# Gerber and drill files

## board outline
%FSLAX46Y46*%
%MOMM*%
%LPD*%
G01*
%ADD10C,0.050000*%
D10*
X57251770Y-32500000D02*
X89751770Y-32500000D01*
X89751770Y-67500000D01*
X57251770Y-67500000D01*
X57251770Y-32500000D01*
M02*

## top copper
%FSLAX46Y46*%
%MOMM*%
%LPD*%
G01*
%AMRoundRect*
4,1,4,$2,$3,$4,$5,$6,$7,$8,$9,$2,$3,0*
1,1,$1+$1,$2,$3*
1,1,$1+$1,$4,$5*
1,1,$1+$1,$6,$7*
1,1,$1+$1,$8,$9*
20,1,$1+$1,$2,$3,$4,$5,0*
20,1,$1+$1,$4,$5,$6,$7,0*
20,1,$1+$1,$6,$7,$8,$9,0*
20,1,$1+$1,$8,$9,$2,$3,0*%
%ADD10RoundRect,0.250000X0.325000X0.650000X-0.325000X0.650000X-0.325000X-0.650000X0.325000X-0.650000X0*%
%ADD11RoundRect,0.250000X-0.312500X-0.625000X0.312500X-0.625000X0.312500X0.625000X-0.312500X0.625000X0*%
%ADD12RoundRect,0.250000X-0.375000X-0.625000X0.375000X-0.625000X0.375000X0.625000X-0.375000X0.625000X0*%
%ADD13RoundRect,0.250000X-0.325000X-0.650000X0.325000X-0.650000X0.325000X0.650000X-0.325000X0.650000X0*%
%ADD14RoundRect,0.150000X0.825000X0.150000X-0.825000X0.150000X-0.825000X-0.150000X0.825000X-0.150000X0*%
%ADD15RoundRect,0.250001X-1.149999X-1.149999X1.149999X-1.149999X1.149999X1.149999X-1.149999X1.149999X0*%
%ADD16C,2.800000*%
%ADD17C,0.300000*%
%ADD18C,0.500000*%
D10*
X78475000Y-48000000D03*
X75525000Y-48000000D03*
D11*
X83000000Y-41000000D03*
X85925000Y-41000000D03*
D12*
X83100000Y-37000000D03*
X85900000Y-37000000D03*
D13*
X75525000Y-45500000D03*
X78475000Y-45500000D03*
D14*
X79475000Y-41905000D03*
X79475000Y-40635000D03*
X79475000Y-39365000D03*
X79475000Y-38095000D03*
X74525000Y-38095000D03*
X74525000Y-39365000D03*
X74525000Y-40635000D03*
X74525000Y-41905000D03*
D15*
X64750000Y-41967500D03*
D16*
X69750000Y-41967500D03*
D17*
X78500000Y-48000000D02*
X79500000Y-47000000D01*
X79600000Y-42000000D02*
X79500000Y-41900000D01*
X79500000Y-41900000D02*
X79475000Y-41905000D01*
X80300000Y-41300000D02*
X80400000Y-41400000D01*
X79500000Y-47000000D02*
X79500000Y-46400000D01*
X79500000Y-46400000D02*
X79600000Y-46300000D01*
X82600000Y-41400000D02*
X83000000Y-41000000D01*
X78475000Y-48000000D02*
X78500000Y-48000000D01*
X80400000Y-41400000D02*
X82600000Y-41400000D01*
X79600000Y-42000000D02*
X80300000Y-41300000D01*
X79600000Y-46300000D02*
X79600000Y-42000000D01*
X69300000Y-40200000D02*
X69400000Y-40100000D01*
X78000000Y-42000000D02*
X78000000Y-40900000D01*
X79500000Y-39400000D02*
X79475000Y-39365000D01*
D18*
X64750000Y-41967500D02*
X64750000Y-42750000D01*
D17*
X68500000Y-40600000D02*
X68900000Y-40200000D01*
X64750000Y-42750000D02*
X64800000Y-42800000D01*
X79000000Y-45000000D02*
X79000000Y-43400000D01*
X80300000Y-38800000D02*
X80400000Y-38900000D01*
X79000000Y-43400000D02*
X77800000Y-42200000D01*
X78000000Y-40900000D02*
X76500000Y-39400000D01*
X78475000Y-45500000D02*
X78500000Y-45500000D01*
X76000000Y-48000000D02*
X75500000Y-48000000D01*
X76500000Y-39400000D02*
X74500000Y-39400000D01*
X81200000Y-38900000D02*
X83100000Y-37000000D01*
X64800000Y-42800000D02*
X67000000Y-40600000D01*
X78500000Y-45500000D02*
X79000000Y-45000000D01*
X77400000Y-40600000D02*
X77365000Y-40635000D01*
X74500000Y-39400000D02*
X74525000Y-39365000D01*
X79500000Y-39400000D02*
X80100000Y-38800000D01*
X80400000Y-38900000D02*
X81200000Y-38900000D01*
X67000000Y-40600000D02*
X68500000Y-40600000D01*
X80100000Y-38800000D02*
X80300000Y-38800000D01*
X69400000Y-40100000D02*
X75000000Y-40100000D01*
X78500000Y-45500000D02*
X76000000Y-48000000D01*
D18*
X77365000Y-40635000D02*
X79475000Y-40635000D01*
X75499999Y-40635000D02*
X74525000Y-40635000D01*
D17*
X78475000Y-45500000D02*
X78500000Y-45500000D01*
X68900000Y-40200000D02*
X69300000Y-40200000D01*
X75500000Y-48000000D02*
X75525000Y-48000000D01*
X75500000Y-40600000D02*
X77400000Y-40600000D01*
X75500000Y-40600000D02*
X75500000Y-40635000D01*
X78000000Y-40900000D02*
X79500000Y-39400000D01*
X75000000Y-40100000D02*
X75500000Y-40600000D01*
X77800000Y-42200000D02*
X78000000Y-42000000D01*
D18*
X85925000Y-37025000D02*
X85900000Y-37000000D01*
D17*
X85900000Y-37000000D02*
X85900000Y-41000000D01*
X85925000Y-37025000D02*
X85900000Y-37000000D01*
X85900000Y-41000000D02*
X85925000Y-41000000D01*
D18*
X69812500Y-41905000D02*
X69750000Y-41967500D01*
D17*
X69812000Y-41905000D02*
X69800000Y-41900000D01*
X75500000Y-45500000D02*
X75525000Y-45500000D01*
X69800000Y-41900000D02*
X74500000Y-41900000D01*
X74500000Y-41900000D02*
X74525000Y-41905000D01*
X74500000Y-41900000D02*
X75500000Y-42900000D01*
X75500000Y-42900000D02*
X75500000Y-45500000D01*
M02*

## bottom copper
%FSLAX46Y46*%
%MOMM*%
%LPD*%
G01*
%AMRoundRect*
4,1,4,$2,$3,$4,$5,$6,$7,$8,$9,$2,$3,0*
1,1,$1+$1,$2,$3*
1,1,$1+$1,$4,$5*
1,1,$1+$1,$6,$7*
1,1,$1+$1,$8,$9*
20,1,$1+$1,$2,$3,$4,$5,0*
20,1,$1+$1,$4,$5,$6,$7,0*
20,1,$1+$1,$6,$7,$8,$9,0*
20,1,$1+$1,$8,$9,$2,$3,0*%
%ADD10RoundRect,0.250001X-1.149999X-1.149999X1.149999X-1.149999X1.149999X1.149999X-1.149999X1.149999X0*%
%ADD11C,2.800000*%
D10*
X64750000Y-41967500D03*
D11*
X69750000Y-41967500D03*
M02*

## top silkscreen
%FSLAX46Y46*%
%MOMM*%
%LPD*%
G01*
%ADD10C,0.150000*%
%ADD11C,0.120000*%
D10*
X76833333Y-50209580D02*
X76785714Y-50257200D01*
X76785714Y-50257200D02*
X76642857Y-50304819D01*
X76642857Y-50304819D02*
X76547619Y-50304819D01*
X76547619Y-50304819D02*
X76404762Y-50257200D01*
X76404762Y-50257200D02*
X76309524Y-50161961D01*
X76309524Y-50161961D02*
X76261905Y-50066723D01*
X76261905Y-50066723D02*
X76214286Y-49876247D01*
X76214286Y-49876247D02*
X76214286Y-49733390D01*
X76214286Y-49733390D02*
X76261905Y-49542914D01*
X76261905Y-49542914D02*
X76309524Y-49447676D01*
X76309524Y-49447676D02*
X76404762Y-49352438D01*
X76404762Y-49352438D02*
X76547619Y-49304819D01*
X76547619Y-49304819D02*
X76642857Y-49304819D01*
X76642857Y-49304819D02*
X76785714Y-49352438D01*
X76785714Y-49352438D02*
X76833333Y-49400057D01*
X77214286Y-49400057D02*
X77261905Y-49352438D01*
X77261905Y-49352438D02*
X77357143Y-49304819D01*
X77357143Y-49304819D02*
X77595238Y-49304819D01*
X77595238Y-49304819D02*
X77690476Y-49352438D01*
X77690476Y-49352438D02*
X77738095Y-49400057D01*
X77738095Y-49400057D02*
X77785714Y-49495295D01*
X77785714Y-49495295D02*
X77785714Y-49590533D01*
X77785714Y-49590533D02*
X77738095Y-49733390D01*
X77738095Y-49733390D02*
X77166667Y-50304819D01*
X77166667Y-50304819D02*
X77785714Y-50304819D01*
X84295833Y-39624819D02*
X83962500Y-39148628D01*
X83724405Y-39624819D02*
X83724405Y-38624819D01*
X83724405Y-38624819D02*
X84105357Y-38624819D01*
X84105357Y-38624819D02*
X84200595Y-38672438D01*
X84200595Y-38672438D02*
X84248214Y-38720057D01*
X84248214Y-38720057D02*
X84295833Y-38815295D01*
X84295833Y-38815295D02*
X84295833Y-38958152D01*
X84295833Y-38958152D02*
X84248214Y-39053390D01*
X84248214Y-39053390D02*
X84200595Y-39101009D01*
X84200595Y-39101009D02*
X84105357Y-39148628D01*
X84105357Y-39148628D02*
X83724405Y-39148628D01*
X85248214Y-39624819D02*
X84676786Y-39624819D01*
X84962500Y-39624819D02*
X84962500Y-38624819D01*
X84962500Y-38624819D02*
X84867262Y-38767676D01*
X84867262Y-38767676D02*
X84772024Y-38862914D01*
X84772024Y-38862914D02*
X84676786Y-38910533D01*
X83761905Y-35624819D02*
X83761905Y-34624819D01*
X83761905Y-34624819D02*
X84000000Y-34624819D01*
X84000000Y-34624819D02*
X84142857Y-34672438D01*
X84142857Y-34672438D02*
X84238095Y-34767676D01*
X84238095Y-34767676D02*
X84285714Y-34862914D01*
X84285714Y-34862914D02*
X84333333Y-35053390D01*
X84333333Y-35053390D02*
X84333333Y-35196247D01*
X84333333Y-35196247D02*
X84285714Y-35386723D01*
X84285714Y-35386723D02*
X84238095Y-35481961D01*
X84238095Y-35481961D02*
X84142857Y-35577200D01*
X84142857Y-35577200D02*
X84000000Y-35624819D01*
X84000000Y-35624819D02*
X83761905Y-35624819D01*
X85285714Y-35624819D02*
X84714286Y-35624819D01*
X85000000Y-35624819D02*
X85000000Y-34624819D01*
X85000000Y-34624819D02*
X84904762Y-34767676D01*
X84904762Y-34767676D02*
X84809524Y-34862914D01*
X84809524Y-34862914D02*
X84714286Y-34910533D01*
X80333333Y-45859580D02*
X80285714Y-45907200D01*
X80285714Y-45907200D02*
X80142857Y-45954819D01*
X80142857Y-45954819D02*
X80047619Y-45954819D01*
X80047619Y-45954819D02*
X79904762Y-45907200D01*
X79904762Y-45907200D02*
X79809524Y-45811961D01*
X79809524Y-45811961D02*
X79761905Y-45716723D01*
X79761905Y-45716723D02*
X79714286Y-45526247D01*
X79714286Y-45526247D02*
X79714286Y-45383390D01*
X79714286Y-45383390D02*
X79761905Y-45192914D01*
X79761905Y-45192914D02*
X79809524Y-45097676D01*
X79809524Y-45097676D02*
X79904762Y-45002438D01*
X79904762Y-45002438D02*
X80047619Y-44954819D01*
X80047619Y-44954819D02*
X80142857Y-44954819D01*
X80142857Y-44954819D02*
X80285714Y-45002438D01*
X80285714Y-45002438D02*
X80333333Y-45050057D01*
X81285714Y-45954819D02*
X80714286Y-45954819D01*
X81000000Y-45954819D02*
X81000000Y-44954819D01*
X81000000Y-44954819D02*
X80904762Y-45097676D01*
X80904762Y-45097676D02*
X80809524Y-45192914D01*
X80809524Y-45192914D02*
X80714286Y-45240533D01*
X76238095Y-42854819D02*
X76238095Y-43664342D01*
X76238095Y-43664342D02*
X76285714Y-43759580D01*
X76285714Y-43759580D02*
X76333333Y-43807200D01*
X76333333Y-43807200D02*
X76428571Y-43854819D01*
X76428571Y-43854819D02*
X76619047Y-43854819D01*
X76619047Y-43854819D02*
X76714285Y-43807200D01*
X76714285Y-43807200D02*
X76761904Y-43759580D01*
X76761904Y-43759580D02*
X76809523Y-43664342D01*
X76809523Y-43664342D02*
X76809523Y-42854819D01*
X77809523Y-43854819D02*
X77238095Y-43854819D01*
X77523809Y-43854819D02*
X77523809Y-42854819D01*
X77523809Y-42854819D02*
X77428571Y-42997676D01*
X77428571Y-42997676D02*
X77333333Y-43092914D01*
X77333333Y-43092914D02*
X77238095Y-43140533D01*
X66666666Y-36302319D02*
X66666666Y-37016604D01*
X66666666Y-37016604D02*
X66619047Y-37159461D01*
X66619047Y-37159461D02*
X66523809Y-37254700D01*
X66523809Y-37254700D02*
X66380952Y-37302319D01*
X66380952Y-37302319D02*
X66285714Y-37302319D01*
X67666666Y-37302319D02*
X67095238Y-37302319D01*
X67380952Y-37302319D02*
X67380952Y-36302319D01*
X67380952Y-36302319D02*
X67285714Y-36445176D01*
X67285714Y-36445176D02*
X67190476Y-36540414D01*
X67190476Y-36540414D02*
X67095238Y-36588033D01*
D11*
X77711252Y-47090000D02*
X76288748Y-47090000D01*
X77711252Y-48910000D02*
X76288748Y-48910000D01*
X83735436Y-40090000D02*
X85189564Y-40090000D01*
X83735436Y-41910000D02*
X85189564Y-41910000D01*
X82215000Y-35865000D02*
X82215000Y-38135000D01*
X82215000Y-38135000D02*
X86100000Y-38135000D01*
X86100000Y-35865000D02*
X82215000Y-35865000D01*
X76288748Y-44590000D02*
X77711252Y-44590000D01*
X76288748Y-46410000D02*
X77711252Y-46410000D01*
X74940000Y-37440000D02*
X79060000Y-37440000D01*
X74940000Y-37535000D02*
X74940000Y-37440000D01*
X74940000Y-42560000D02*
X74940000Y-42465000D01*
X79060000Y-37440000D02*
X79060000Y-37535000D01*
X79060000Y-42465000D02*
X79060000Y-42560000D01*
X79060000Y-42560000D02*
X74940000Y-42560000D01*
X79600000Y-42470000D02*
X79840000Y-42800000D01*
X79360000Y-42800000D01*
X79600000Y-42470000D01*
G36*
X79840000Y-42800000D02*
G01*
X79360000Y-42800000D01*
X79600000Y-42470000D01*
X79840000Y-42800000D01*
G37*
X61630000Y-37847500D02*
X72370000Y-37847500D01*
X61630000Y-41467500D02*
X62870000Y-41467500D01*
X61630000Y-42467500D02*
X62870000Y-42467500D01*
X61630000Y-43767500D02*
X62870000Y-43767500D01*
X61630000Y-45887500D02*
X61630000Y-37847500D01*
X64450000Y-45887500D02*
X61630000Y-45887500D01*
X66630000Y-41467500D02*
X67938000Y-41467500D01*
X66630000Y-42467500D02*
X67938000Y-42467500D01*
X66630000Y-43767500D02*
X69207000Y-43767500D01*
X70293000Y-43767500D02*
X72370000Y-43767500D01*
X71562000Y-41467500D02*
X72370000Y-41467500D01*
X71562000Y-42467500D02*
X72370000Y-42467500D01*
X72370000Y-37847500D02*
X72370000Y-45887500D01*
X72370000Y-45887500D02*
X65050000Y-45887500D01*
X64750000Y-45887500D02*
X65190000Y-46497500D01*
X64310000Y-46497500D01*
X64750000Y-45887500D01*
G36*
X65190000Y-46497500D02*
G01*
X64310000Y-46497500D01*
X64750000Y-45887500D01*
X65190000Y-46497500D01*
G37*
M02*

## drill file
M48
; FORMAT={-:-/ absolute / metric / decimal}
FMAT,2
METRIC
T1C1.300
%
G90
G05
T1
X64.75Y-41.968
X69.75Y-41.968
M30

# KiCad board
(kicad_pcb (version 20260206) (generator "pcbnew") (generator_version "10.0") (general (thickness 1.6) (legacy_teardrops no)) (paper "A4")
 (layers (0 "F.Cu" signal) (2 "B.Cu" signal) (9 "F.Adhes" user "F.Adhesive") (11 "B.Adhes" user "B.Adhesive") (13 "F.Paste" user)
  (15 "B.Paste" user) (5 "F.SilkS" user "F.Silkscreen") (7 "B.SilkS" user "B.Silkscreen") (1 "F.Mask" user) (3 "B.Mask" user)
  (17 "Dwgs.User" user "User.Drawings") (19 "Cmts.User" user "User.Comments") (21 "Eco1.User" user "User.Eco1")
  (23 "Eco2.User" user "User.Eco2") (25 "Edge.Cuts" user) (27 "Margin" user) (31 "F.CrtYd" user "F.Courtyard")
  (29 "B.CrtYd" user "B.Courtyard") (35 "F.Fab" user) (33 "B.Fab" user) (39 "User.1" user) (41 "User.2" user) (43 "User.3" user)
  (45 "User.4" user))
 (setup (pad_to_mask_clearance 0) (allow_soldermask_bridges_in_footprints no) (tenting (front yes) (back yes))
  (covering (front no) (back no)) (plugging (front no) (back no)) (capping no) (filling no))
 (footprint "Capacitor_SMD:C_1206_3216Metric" (layer "F.Cu") (at 77 48 180)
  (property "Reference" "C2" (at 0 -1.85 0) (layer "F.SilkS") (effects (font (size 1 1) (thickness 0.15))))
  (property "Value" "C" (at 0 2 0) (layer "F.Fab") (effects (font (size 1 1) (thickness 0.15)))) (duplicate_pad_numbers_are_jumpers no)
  (fp_line (start -0.711252 0.91) (end 0.711252 0.91) (stroke (width 0.12) (type solid)) (layer "F.SilkS"))
  (fp_line (start -0.711252 -0.91) (end 0.711252 -0.91) (stroke (width 0.12) (type solid)) (layer "F.SilkS"))
  (pad "1" smd roundrect (at -1.475 0 180) (size 1.15 1.8) (layers "F.Cu" "F.Mask" "F.Paste") (roundrect_rratio 0.217391)
   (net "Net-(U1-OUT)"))
  (pad "2" smd roundrect (at 1.475 0 180) (size 1.15 1.8) (layers "F.Cu" "F.Mask" "F.Paste") (roundrect_rratio 0.217391) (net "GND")))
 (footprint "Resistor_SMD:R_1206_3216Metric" (layer "F.Cu") (at 84.4625 41)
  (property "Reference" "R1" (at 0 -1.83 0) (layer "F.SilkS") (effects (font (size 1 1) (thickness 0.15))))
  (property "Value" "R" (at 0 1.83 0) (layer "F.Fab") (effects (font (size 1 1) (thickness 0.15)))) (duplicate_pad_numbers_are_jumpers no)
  (fp_line (start -0.727064 -0.91) (end 0.727064 -0.91) (stroke (width 0.12) (type solid)) (layer "F.SilkS"))
  (fp_line (start -0.727064 0.91) (end 0.727064 0.91) (stroke (width 0.12) (type solid)) (layer "F.SilkS"))
  (pad "1" smd roundrect (at -1.4625 0) (size 1.125 1.75) (layers "F.Cu" "F.Mask" "F.Paste") (roundrect_rratio 0.222222)
   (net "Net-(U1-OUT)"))
  (pad "2" smd roundrect (at 1.4625 0) (size 1.125 1.75) (layers "F.Cu" "F.Mask" "F.Paste") (roundrect_rratio 0.222222) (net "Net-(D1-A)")))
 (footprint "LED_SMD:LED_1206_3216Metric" (layer "F.Cu") (at 84.5 37)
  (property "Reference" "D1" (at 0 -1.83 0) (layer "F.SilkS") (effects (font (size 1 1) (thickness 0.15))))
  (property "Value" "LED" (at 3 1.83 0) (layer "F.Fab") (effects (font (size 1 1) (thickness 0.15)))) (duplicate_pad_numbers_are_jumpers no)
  (fp_line (start -2.285 -1.135) (end -2.285 1.135) (stroke (width 0.12) (type solid)) (layer "F.SilkS"))
  (fp_line (start -2.285 1.135) (end 1.6 1.135) (stroke (width 0.12) (type solid)) (layer "F.SilkS"))
  (fp_line (start 1.6 -1.135) (end -2.285 -1.135) (stroke (width 0.12) (type solid)) (layer "F.SilkS"))
  (pad "1" smd roundrect (at -1.4 0) (size 1.25 1.75) (layers "F.Cu" "F.Mask" "F.Paste") (roundrect_rratio 0.2) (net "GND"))
  (pad "2" smd roundrect (at 1.4 0) (size 1.25 1.75) (layers "F.Cu" "F.Mask" "F.Paste") (roundrect_rratio 0.2) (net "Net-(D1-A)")))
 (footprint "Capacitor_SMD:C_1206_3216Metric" (layer "F.Cu") (at 77 45.5)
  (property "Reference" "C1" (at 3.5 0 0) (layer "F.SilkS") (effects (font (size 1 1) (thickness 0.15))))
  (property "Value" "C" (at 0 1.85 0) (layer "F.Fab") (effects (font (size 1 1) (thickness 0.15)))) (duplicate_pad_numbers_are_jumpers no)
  (fp_line (start -0.711252 -0.91) (end 0.711252 -0.91) (stroke (width 0.12) (type solid)) (layer "F.SilkS"))
  (fp_line (start -0.711252 0.91) (end 0.711252 0.91) (stroke (width 0.12) (type solid)) (layer "F.SilkS"))
  (pad "1" smd roundrect (at -1.475 0) (size 1.15 1.8) (layers "F.Cu" "F.Mask" "F.Paste") (roundrect_rratio 0.217391) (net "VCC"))
  (pad "2" smd roundrect (at 1.475 0) (size 1.15 1.8) (layers "F.Cu" "F.Mask" "F.Paste") (roundrect_rratio 0.217391) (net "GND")))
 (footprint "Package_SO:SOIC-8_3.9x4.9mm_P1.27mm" (layer "F.Cu") (at 77 40 180)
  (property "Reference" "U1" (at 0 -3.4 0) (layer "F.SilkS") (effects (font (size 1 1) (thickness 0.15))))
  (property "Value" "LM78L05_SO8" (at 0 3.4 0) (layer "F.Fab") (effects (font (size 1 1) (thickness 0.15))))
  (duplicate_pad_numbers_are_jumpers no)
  (fp_line (start 2.06 2.56) (end -2.06 2.56) (stroke (width 0.12) (type solid)) (layer "F.SilkS"))
  (fp_line (start 2.06 2.465) (end 2.06 2.56) (stroke (width 0.12) (type solid)) (layer "F.SilkS"))
  (fp_line (start 2.06 -2.56) (end 2.06 -2.465) (stroke (width 0.12) (type solid)) (layer "F.SilkS"))
  (fp_line (start -2.06 2.56) (end -2.06 2.465) (stroke (width 0.12) (type solid)) (layer "F.SilkS"))
  (fp_line (start -2.06 -2.465) (end -2.06 -2.56) (stroke (width 0.12) (type solid)) (layer "F.SilkS"))
  (fp_line (start -2.06 -2.56) (end 2.06 -2.56) (stroke (width 0.12) (type solid)) (layer "F.SilkS"))
  (fp_poly (pts (xy -2.6 -2.47) (xy -2.84 -2.8) (xy -2.36 -2.8)) (stroke (width 0.12) (type solid)) (fill yes) (layer "F.SilkS"))
  (pad "1" smd roundrect (at -2.475 -1.905 180) (size 1.95 0.6) (layers "F.Cu" "F.Mask" "F.Paste") (roundrect_rratio 0.25)
   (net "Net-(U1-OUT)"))
  (pad "2" smd roundrect (at -2.475 -0.635 180) (size 1.95 0.6) (layers "F.Cu" "F.Mask" "F.Paste") (roundrect_rratio 0.25) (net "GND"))
  (pad "3" smd roundrect (at -2.475 0.635 180) (size 1.95 0.6) (layers "F.Cu" "F.Mask" "F.Paste") (roundrect_rratio 0.25) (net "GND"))
  (pad "4" smd roundrect (at -2.475 1.905 180) (size 1.95 0.6) (layers "F.Cu" "F.Mask" "F.Paste") (roundrect_rratio 0.25)
   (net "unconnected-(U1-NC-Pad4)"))
  (pad "5" smd roundrect (at 2.475 1.905 180) (size 1.95 0.6) (layers "F.Cu" "F.Mask" "F.Paste") (roundrect_rratio 0.25)
   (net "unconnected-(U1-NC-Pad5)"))
  (pad "6" smd roundrect (at 2.475 0.635 180) (size 1.95 0.6) (layers "F.Cu" "F.Mask" "F.Paste") (roundrect_rratio 0.25) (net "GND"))
  (pad "7" smd roundrect (at 2.475 -0.635 180) (size 1.95 0.6) (layers "F.Cu" "F.Mask" "F.Paste") (roundrect_rratio 0.25) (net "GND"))
  (pad "8" smd roundrect (at 2.475 -1.905 180) (size 1.95 0.6) (layers "F.Cu" "F.Mask" "F.Paste") (roundrect_rratio 0.25) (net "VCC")))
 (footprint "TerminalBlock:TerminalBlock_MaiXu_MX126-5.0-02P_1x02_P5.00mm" (layer "F.Cu") (at 64.75 41.9675)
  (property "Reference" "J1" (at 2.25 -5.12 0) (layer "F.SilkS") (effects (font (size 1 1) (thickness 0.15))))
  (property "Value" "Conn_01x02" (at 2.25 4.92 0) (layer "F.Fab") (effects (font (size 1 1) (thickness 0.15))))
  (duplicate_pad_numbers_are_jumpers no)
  (fp_line (start -3.12 -4.12) (end 7.62 -4.12) (stroke (width 0.12) (type solid)) (layer "F.SilkS"))
  (fp_line (start -3.12 -0.5) (end -1.88 -0.5) (stroke (width 0.12) (type solid)) (layer "F.SilkS"))
  (fp_line (start -3.12 0.5) (end -1.88 0.5) (stroke (width 0.12) (type solid)) (layer "F.SilkS"))
  (fp_line (start -3.12 1.8) (end -1.88 1.8) (stroke (width 0.12) (type solid)) (layer "F.SilkS"))
  (fp_line (start -3.12 3.92) (end -3.12 -4.12) (stroke (width 0.12) (type solid)) (layer "F.SilkS"))
  (fp_line (start -0.3 3.92) (end -3.12 3.92) (stroke (width 0.12) (type solid)) (layer "F.SilkS"))
  (fp_line (start 1.88 -0.5) (end 3.188 -0.5) (stroke (width 0.12) (type solid)) (layer "F.SilkS"))
  (fp_line (start 1.88 0.5) (end 3.188 0.5) (stroke (width 0.12) (type solid)) (layer "F.SilkS"))
  (fp_line (start 1.88 1.8) (end 4.457 1.8) (stroke (width 0.12) (type solid)) (layer "F.SilkS"))
  (fp_line (start 5.543 1.8) (end 7.62 1.8) (stroke (width 0.12) (type solid)) (layer "F.SilkS"))
  (fp_line (start 6.812 -0.5) (end 7.62 -0.5) (stroke (width 0.12) (type solid)) (layer "F.SilkS"))
  (fp_line (start 6.812 0.5) (end 7.62 0.5) (stroke (width 0.12) (type solid)) (layer "F.SilkS"))
  (fp_line (start 7.62 -4.12) (end 7.62 3.92) (stroke (width 0.12) (type solid)) (layer "F.SilkS"))
  (fp_line (start 7.62 3.92) (end 0.3 3.92) (stroke (width 0.12) (type solid)) (layer "F.SilkS"))
  (fp_poly (pts (xy 0 3.92) (xy 0.44 4.53) (xy -0.44 4.53)) (stroke (width 0.12) (type solid)) (fill yes) (layer "F.SilkS"))
  (pad "1" thru_hole roundrect (at 0 0) (size 2.8 2.8) (drill 1.3) (layers "*.Cu" "*.Mask") (remove_unused_layers no)
   (roundrect_rratio 0.089286) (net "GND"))
  (pad "2" thru_hole circle (at 5 0) (size 2.8 2.8) (drill 1.3) (layers "*.Cu" "*.Mask") (remove_unused_layers no) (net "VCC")))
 (gr_poly
  (pts (xy 57.25177 32.5) (xy 89.75177 32.5) (xy 89.75177 67.5) (xy 57.25177 67.5)) (stroke (width 0.05) (type solid)) (fill no)
  (layer "Edge.Cuts"))
 (segment (start 78.5 48) (end 79.5 47) (width 0.3) (layer "F.Cu") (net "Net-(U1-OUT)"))
 (segment (start 79.6 42) (end 79.5 41.9) (width 0.3) (layer "F.Cu") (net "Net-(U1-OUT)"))
 (segment (start 79.5 41.9) (end 79.475 41.905) (width 0.3) (layer "F.Cu") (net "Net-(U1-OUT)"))
 (segment (start 80.3 41.3) (end 80.4 41.4) (width 0.3) (layer "F.Cu") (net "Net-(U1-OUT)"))
 (segment (start 79.5 47) (end 79.5 46.4) (width 0.3) (layer "F.Cu") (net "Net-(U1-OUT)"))
 (segment (start 79.5 46.4) (end 79.6 46.3) (width 0.3) (layer "F.Cu") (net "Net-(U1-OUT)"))
 (segment (start 82.6 41.4) (end 83 41) (width 0.3) (layer "F.Cu") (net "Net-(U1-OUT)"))
 (segment (start 78.475 48) (end 78.5 48) (width 0.3) (layer "F.Cu") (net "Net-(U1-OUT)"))
 (segment (start 80.4 41.4) (end 82.6 41.4) (width 0.3) (layer "F.Cu") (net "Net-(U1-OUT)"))
 (segment (start 79.6 42) (end 80.3 41.3) (width 0.3) (layer "F.Cu") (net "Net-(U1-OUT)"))
 (segment (start 79.6 46.3) (end 79.6 42) (width 0.3) (layer "F.Cu") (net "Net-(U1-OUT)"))
 (segment (start 69.3 40.2) (end 69.4 40.1) (width 0.3) (layer "F.Cu") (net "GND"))
 (segment (start 78 42) (end 78 40.9) (width 0.3) (layer "F.Cu") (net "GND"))
 (segment (start 79.5 39.4) (end 79.475 39.365) (width 0.3) (layer "F.Cu") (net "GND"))
 (segment (start 64.75 41.9675) (end 64.75 42.75) (width 0.5) (layer "F.Cu") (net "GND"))
 (segment (start 68.5 40.6) (end 68.9 40.2) (width 0.3) (layer "F.Cu") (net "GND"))
 (segment (start 64.75 42.75) (end 64.8 42.8) (width 0.3) (layer "F.Cu") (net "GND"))
 (segment (start 79 45) (end 79 43.4) (width 0.3) (layer "F.Cu") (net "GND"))
 (segment (start 80.3 38.8) (end 80.4 38.9) (width 0.3) (layer "F.Cu") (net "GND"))
 (segment (start 79 43.4) (end 77.8 42.2) (width 0.3) (layer "F.Cu") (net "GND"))
 (segment (start 78 40.9) (end 76.5 39.4) (width 0.3) (layer "F.Cu") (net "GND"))
 (segment (start 78.475 45.5) (end 78.5 45.5) (width 0.3) (layer "F.Cu") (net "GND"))
 (segment (start 76 48) (end 75.5 48) (width 0.3) (layer "F.Cu") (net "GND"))
 (segment (start 76.5 39.4) (end 74.5 39.4) (width 0.3) (layer "F.Cu") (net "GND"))
 (segment (start 81.2 38.9) (end 83.1 37) (width 0.3) (layer "F.Cu") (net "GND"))
 (segment (start 64.8 42.8) (end 67 40.6) (width 0.3) (layer "F.Cu") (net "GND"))
 (segment (start 78.5 45.5) (end 79 45) (width 0.3) (layer "F.Cu") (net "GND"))
 (segment (start 77.4 40.6) (end 77.365 40.635) (width 0.3) (layer "F.Cu") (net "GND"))
 (segment (start 74.5 39.4) (end 74.525 39.365) (width 0.3) (layer "F.Cu") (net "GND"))
 (segment (start 79.5 39.4) (end 80.1 38.8) (width 0.3) (layer "F.Cu") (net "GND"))
 (segment (start 80.4 38.9) (end 81.2 38.9) (width 0.3) (layer "F.Cu") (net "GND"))
 (segment (start 67 40.6) (end 68.5 40.6) (width 0.3) (layer "F.Cu") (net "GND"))
 (segment (start 80.1 38.8) (end 80.3 38.8) (width 0.3) (layer "F.Cu") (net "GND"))
 (segment (start 69.4 40.1) (end 75 40.1) (width 0.3) (layer "F.Cu") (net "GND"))
 (segment (start 78.5 45.5) (end 76 48) (width 0.3) (layer "F.Cu") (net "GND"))
 (segment (start 77.365 40.635) (end 79.475 40.635) (width 0.5) (layer "F.Cu") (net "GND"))
 (segment (start 75.499999 40.635) (end 74.525 40.635) (width 0.5) (layer "F.Cu") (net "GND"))
 (segment (start 78.475 45.5) (end 78.5 45.5) (width 0.3) (layer "F.Cu") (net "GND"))
 (segment (start 68.9 40.2) (end 69.3 40.2) (width 0.3) (layer "F.Cu") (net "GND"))
 (segment (start 75.5 48) (end 75.525 48) (width 0.3) (layer "F.Cu") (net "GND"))
 (segment (start 75.5 40.6) (end 77.4 40.6) (width 0.3) (layer "F.Cu") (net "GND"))
 (segment (start 75.5 40.6) (end 75.5 40.635) (width 0.3) (layer "F.Cu") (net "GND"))
 (segment (start 78 40.9) (end 79.5 39.4) (width 0.3) (layer "F.Cu") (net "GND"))
 (segment (start 75 40.1) (end 75.5 40.6) (width 0.3) (layer "F.Cu") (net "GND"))
 (segment (start 77.8 42.2) (end 78 42) (width 0.3) (layer "F.Cu") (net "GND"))
 (segment (start 85.925 37.025) (end 85.9 37) (width 0.5) (layer "F.Cu") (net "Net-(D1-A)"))
 (segment (start 85.9 37) (end 85.9 41) (width 0.3) (layer "F.Cu") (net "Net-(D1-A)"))
 (segment (start 85.925 37.025) (end 85.9 37) (width 0.3) (layer "F.Cu") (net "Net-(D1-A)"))
 (segment (start 85.9 41) (end 85.925 41) (width 0.3) (layer "F.Cu") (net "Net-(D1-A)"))
 (segment (start 69.8125 41.905) (end 69.75 41.9675) (width 0.5) (layer "F.Cu") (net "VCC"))
 (segment (start 69.812 41.905) (end 69.8 41.9) (width 0.3) (layer "F.Cu") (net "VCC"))
 (segment (start 75.5 45.5) (end 75.525 45.5) (width 0.3) (layer "F.Cu") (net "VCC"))
 (segment (start 69.8 41.9) (end 74.5 41.9) (width 0.3) (layer "F.Cu") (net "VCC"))
 (segment (start 74.5 41.9) (end 74.525 41.905) (width 0.3) (layer "F.Cu") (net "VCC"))
 (segment (start 74.5 41.9) (end 75.5 42.9) (width 0.3) (layer "F.Cu") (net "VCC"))
 (segment (start 75.5 42.9) (end 75.5 45.5) (width 0.3) (layer "F.Cu") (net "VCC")))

